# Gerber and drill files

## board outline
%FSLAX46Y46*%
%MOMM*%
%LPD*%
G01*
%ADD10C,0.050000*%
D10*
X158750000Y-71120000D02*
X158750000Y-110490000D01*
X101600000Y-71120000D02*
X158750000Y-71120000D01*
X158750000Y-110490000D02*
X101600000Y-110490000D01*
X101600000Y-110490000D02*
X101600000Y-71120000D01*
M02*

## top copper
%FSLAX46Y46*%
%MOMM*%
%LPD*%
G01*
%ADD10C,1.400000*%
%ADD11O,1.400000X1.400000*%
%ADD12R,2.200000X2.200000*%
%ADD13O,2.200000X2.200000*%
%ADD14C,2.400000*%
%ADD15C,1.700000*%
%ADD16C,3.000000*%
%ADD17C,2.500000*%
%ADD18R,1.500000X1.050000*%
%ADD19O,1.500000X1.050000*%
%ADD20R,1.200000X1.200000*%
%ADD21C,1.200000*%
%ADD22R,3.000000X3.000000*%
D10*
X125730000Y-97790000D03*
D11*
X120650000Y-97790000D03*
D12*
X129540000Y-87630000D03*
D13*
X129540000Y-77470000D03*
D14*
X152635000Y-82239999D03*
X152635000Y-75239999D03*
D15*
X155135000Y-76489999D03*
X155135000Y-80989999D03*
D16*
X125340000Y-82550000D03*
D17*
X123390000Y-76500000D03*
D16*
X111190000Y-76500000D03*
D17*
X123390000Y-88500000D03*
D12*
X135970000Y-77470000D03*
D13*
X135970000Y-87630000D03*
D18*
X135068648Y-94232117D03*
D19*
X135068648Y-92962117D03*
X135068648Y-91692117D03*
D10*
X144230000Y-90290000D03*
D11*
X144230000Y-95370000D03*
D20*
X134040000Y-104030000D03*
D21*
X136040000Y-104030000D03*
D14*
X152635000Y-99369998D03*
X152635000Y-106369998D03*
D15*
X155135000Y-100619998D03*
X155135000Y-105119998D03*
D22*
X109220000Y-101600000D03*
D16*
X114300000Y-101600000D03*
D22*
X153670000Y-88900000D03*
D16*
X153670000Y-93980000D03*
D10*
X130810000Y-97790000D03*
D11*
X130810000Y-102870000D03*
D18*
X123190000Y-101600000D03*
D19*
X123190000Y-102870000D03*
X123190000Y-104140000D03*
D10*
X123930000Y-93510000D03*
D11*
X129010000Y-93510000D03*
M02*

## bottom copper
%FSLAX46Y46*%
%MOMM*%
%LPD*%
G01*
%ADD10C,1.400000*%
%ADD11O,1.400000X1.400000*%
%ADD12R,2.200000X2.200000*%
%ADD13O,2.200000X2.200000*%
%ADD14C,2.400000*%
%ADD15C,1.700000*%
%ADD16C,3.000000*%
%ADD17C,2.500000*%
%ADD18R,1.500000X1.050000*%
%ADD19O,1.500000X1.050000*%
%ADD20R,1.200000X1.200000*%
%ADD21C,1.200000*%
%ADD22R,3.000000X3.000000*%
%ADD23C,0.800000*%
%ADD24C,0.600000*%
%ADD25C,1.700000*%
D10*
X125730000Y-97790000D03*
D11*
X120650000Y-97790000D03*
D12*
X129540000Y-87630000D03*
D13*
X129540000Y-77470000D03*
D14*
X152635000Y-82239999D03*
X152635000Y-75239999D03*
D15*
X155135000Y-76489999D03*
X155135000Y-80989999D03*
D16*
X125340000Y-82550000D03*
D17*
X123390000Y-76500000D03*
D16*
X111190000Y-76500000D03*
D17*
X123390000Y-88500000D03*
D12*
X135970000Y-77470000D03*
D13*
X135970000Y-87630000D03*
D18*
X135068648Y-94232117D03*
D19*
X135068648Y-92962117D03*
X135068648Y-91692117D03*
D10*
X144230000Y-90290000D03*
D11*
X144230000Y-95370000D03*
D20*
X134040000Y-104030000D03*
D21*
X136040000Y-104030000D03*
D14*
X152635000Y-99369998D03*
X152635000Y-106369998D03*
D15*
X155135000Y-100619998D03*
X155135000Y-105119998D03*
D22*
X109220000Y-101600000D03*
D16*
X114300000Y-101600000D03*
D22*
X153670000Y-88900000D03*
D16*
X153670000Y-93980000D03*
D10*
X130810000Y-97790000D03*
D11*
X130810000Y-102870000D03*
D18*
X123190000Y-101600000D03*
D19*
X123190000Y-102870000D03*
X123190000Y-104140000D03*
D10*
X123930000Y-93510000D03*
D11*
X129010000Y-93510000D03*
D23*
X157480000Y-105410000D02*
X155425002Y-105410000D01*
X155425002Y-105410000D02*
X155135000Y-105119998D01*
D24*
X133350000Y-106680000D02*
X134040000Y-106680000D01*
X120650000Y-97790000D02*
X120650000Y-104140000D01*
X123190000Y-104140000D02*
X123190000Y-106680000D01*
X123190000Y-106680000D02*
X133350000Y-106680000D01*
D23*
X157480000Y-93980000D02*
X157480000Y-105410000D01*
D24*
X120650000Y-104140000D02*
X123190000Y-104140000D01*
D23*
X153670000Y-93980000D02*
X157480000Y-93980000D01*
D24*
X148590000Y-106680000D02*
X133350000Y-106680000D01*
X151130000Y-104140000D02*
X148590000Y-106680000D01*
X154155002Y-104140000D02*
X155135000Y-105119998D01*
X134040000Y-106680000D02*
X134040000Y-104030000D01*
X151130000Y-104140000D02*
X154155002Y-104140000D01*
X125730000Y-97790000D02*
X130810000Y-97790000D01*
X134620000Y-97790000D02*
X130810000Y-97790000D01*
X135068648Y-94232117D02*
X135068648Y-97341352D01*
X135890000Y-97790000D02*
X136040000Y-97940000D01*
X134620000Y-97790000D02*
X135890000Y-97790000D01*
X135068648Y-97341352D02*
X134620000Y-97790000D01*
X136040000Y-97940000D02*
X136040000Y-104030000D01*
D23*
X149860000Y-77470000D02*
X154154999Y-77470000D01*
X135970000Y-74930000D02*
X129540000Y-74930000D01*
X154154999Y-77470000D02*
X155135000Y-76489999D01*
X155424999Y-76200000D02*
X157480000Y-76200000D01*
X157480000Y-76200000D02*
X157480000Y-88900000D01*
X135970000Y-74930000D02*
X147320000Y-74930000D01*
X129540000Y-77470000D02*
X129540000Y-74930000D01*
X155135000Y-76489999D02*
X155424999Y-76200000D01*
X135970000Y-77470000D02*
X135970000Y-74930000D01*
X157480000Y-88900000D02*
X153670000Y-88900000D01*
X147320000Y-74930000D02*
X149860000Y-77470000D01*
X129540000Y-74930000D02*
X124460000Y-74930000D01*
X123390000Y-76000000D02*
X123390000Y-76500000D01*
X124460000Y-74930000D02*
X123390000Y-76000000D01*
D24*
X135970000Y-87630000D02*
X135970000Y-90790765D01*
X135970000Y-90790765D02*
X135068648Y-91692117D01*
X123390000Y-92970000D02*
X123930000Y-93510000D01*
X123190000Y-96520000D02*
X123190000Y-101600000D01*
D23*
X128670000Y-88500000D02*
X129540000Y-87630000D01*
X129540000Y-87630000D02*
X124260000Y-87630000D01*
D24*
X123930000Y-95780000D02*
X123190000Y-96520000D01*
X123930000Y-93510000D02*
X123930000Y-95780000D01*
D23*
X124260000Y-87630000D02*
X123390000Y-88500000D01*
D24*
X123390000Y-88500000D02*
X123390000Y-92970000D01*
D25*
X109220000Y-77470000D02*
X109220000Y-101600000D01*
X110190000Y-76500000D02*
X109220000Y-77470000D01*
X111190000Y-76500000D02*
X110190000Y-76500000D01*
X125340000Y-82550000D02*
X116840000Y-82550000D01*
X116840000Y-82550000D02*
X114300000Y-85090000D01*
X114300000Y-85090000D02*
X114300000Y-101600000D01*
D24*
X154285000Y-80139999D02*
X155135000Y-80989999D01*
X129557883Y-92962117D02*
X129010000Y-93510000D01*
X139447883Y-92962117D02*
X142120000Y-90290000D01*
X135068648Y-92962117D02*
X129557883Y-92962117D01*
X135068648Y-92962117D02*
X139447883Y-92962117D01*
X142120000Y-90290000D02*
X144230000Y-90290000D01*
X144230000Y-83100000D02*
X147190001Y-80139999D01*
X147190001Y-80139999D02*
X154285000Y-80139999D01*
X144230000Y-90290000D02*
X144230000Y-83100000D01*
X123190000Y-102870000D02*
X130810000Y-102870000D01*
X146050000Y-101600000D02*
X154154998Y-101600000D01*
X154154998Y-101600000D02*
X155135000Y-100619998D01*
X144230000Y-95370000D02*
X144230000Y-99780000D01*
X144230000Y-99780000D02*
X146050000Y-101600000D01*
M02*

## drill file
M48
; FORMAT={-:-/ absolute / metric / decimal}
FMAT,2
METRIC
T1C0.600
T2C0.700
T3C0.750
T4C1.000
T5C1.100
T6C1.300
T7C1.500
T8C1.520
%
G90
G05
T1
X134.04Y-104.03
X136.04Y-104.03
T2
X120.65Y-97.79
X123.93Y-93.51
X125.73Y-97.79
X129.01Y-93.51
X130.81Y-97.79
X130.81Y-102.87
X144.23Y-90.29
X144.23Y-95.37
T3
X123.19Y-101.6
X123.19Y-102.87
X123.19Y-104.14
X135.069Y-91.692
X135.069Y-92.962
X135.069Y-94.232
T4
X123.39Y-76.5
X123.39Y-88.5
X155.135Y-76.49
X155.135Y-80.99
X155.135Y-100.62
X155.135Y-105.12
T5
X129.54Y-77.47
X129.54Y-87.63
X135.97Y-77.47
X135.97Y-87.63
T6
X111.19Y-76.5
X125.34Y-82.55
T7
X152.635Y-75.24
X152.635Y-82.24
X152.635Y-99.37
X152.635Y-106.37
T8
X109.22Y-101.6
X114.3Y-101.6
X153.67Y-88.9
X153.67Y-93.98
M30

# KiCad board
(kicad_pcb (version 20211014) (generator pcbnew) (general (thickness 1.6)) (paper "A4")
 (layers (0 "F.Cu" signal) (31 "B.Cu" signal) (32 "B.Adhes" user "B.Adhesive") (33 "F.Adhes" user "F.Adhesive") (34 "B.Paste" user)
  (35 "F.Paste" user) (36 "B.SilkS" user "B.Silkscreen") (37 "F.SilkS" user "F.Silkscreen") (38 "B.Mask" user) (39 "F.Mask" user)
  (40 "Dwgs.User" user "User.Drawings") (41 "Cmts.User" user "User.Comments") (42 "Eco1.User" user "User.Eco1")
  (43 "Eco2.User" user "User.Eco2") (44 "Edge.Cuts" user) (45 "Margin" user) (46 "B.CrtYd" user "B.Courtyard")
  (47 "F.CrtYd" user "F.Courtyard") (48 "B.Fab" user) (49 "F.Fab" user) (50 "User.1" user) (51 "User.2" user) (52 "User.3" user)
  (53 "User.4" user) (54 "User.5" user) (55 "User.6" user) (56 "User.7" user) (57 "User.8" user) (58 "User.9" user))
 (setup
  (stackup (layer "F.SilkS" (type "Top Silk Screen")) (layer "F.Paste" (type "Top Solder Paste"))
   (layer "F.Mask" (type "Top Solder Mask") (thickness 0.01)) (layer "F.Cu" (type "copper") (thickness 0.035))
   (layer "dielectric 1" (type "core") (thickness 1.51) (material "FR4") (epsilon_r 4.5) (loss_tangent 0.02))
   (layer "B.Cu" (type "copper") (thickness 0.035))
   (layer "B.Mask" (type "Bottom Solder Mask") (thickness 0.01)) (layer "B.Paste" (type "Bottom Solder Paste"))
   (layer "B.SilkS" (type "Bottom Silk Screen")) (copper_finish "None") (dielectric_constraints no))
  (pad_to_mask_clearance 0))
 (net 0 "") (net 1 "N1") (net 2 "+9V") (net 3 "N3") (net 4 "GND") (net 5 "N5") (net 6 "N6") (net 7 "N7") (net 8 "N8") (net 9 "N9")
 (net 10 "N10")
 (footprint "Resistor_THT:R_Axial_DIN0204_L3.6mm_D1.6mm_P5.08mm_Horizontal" (layer "F.Cu") (at 125.73 97.79 180)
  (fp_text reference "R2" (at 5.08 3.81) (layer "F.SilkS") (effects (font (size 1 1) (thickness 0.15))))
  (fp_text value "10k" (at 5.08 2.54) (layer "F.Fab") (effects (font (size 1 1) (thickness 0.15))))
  (pad "1" thru_hole circle (at 0 0 180) (size 1.4 1.4) (drill 0.7) (layers *.Cu *.Mask) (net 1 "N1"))
  (pad "2" thru_hole oval (at 5.08 0 180) (size 1.4 1.4) (drill 0.7) (layers *.Cu *.Mask) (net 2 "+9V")))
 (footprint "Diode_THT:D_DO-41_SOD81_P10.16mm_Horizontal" (layer "F.Cu") (at 129.54 87.63 90)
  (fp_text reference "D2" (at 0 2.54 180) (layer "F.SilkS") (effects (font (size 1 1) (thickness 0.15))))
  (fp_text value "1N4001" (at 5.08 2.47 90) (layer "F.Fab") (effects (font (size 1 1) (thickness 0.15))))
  (pad "1" thru_hole rect (at 0 0 90) (size 2.2 2.2) (drill 1.1) (layers *.Cu *.Mask) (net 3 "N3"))
  (pad "2" thru_hole oval (at 10.16 0 90) (size 2.2 2.2) (drill 1.1) (layers *.Cu *.Mask) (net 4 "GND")))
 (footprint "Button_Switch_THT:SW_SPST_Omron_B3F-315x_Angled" (layer "F.Cu") (at 155.135 76.489999 -90)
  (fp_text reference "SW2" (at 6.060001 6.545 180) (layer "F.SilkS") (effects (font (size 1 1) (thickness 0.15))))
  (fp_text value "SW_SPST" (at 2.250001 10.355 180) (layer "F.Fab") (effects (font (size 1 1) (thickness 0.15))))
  (pad "" thru_hole circle (at 5.75 2.5 90) (size 2.4 2.4) (drill 1.5) (layers *.Cu *.Mask))
  (pad "" thru_hole circle (at -1.25 2.5 90) (size 2.4 2.4) (drill 1.5) (layers *.Cu *.Mask))
  (pad "1" thru_hole circle (at 0 0 90) (size 1.7 1.7) (drill 1) (layers *.Cu *.Mask) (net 4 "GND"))
  (pad "2" thru_hole circle (at 4.5 0 90) (size 1.7 1.7) (drill 1) (layers *.Cu *.Mask) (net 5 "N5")))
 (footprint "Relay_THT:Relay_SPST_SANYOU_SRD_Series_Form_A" (layer "F.Cu") (at 125.34 82.55 180)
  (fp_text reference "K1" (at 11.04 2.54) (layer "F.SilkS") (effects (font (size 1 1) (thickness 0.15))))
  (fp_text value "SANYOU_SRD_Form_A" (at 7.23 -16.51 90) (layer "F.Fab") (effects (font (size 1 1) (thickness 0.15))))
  (pad "1" thru_hole circle (at 0 0 270) (size 3 3) (drill 1.3) (layers *.Cu *.Mask) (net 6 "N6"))
  (pad "2" thru_hole circle (at 1.95 6.05 270) (size 2.5 2.5) (drill 1) (layers *.Cu *.Mask) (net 4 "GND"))
  (pad "3" thru_hole circle (at 14.15 6.05 270) (size 3 3) (drill 1.3) (layers *.Cu *.Mask) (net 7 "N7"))
  (pad "5" thru_hole circle (at 1.95 -5.95 270) (size 2.5 2.5) (drill 1) (layers *.Cu *.Mask) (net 3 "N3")))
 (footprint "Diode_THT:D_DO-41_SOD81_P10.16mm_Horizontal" (layer "F.Cu") (at 135.97 77.47 -90)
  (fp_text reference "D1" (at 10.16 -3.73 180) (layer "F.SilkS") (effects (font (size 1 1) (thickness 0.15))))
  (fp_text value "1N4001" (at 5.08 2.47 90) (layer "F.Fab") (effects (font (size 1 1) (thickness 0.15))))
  (pad "1" thru_hole rect (at 0 0 270) (size 2.2 2.2) (drill 1.1) (layers *.Cu *.Mask) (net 4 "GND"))
  (pad "2" thru_hole oval (at 10.16 0 270) (size 2.2 2.2) (drill 1.1) (layers *.Cu *.Mask) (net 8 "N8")))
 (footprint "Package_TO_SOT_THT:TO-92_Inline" (layer "F.Cu") (at 135.068648 94.232117 90)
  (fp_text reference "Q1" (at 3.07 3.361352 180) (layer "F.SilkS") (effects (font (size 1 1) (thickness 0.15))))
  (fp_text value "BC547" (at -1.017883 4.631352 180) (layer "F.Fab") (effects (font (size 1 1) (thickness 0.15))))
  (pad "1" thru_hole rect (at 0 0 90) (size 1.05 1.5) (drill 0.75) (layers *.Cu *.Mask) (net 1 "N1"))
  (pad "2" thru_hole oval (at 1.27 0 90) (size 1.05 1.5) (drill 0.75) (layers *.Cu *.Mask) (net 5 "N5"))
  (pad "3" thru_hole oval (at 2.54 0 90) (size 1.05 1.5) (drill 0.75) (layers *.Cu *.Mask) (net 8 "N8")))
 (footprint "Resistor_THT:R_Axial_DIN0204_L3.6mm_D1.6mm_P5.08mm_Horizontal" (layer "F.Cu") (at 144.23 90.29 -90)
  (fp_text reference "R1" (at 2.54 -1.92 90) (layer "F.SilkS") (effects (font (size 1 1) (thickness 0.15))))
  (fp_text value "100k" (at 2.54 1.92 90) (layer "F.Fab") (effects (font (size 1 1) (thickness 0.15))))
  (pad "1" thru_hole circle (at 0 0 270) (size 1.4 1.4) (drill 0.7) (layers *.Cu *.Mask) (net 5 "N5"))
  (pad "2" thru_hole oval (at 5.08 0 270) (size 1.4 1.4) (drill 0.7) (layers *.Cu *.Mask) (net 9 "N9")))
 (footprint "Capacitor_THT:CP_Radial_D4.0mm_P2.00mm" (layer "F.Cu") (at 134.04 104.03)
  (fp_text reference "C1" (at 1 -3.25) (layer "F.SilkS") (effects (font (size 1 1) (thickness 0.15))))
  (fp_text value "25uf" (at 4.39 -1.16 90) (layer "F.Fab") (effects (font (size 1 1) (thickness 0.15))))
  (pad "1" thru_hole rect (at 0 0) (size 1.2 1.2) (drill 0.6) (layers *.Cu *.Mask) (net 2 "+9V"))
  (pad "2" thru_hole circle (at 2 0) (size 1.2 1.2) (drill 0.6) (layers *.Cu *.Mask) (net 1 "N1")))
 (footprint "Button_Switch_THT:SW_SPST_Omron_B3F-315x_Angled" (layer "F.Cu") (at 155.135 100.619998 -90)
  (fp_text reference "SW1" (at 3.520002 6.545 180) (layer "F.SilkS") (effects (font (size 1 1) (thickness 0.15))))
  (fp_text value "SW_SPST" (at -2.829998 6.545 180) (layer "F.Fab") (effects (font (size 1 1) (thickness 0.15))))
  (pad "" thru_hole circle (at -1.25 2.5 90) (size 2.4 2.4) (drill 1.5) (layers *.Cu *.Mask))
  (pad "" thru_hole circle (at 5.75 2.5 90) (size 2.4 2.4) (drill 1.5) (layers *.Cu *.Mask))
  (pad "1" thru_hole circle (at 0 0 90) (size 1.7 1.7) (drill 1) (layers *.Cu *.Mask) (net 9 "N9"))
  (pad "2" thru_hole circle (at 4.5 0 90) (size 1.7 1.7) (drill 1) (layers *.Cu *.Mask) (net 2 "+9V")))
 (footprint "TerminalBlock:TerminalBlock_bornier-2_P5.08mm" (layer "F.Cu") (at 109.22 101.6)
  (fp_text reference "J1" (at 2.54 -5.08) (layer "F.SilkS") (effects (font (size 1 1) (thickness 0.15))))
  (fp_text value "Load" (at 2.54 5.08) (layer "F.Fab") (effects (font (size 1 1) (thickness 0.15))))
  (pad "1" thru_hole rect (at 0 0) (size 3 3) (drill 1.52) (layers *.Cu *.Mask) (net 7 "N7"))
  (pad "2" thru_hole circle (at 5.08 0) (size 3 3) (drill 1.52) (layers *.Cu *.Mask) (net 6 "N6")))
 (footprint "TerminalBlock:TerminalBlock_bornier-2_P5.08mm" (layer "F.Cu") (at 153.67 88.9 -90)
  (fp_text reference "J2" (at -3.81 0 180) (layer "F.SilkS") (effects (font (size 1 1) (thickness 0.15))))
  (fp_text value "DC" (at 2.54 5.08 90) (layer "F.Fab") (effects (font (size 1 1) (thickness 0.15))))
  (pad "1" thru_hole rect (at 0 0 270) (size 3 3) (drill 1.52) (layers *.Cu *.Mask) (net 4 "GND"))
  (pad "2" thru_hole circle (at 5.08 0 270) (size 3 3) (drill 1.52) (layers *.Cu *.Mask) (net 2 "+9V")))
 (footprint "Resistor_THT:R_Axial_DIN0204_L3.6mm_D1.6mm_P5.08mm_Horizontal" (layer "F.Cu") (at 130.81 97.79 -90)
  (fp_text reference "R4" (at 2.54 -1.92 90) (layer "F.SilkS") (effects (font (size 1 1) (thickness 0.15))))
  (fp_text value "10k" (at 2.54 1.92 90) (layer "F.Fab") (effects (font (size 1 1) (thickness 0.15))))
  (pad "1" thru_hole circle (at 0 0 270) (size 1.4 1.4) (drill 0.7) (layers *.Cu *.Mask) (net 1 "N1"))
  (pad "2" thru_hole oval (at 5.08 0 270) (size 1.4 1.4) (drill 0.7) (layers *.Cu *.Mask) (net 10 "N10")))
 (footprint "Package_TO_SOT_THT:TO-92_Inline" (layer "F.Cu") (at 123.19 101.6 -90)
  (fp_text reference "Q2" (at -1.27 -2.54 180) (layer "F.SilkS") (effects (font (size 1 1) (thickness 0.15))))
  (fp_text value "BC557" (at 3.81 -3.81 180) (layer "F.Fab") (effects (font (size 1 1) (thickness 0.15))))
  (pad "1" thru_hole rect (at 0 0 270) (size 1.05 1.5) (drill 0.75) (layers *.Cu *.Mask) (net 3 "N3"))
  (pad "2" thru_hole oval (at 1.27 0 270) (size 1.05 1.5) (drill 0.75) (layers *.Cu *.Mask) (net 10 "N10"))
  (pad "3" thru_hole oval (at 2.54 0 270) (size 1.05 1.5) (drill 0.75) (layers *.Cu *.Mask) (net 2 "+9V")))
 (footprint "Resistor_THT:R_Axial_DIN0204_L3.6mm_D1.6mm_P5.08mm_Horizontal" (layer "F.Cu") (at 123.93 93.51)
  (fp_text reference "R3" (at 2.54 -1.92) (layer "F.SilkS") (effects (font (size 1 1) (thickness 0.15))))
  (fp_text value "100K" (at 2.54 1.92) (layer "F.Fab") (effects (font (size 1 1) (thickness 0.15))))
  (pad "1" thru_hole circle (at 0 0) (size 1.4 1.4) (drill 0.7) (layers *.Cu *.Mask) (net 3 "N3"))
  (pad "2" thru_hole oval (at 5.08 0) (size 1.4 1.4) (drill 0.7) (layers *.Cu *.Mask) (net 5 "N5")))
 (gr_line (start 158.75 71.12) (end 158.75 110.49) (layer "Edge.Cuts") (width 0.05))
 (gr_line (start 101.6 71.12) (end 158.75 71.12) (layer "Edge.Cuts") (width 0.05))
 (gr_line (start 158.75 110.49) (end 101.6 110.49) (layer "Edge.Cuts") (width 0.05))
 (gr_line (start 101.6 110.49) (end 101.6 71.12) (layer "Edge.Cuts") (width 0.05))
 (segment (start 157.48 105.41) (end 155.425002 105.41) (width 0.8) (layer "B.Cu") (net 2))
 (segment (start 155.425002 105.41) (end 155.135 105.119998) (width 0.8) (layer "B.Cu") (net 2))
 (segment (start 133.35 106.68) (end 134.04 106.68) (width 0.6) (layer "B.Cu") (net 2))
 (segment (start 120.65 97.79) (end 120.65 104.14) (width 0.6) (layer "B.Cu") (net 2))
 (segment (start 123.19 104.14) (end 123.19 106.68) (width 0.6) (layer "B.Cu") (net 2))
 (segment (start 123.19 106.68) (end 133.35 106.68) (width 0.6) (layer "B.Cu") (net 2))
 (segment (start 157.48 93.98) (end 157.48 105.41) (width 0.8) (layer "B.Cu") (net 2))
 (segment (start 120.65 104.14) (end 123.19 104.14) (width 0.6) (layer "B.Cu") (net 2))
 (segment (start 153.67 93.98) (end 157.48 93.98) (width 0.8) (layer "B.Cu") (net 2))
 (segment (start 148.59 106.68) (end 133.35 106.68) (width 0.6) (layer "B.Cu") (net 2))
 (segment (start 151.13 104.14) (end 148.59 106.68) (width 0.6) (layer "B.Cu") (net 2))
 (segment (start 154.155002 104.14) (end 155.135 105.119998) (width 0.6) (layer "B.Cu") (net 2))
 (segment (start 134.04 106.68) (end 134.04 104.03) (width 0.6) (layer "B.Cu") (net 2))
 (segment (start 151.13 104.14) (end 154.155002 104.14) (width 0.6) (layer "B.Cu") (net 2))
 (segment (start 125.73 97.79) (end 130.81 97.79) (width 0.6) (layer "B.Cu") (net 1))
 (segment (start 134.62 97.79) (end 130.81 97.79) (width 0.6) (layer "B.Cu") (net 1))
 (segment (start 135.068648 94.232117) (end 135.068648 97.341352) (width 0.6) (layer "B.Cu") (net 1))
 (segment (start 135.89 97.79) (end 136.04 97.94) (width 0.6) (layer "B.Cu") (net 1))
 (segment (start 134.62 97.79) (end 135.89 97.79) (width 0.6) (layer "B.Cu") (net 1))
 (segment (start 135.068648 97.341352) (end 134.62 97.79) (width 0.6) (layer "B.Cu") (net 1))
 (segment (start 136.04 97.94) (end 136.04 104.03) (width 0.6) (layer "B.Cu") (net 1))
 (segment (start 149.86 77.47) (end 154.154999 77.47) (width 0.8) (layer "B.Cu") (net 4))
 (segment (start 135.97 74.93) (end 129.54 74.93) (width 0.8) (layer "B.Cu") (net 4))
 (segment (start 154.154999 77.47) (end 155.135 76.489999) (width 0.8) (layer "B.Cu") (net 4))
 (segment (start 155.424999 76.2) (end 157.48 76.2) (width 0.8) (layer "B.Cu") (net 4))
 (segment (start 157.48 76.2) (end 157.48 88.9) (width 0.8) (layer "B.Cu") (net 4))
 (segment (start 135.97 74.93) (end 147.32 74.93) (width 0.8) (layer "B.Cu") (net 4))
 (segment (start 129.54 77.47) (end 129.54 74.93) (width 0.8) (layer "B.Cu") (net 4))
 (segment (start 155.135 76.489999) (end 155.424999 76.2) (width 0.8) (layer "B.Cu") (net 4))
 (segment (start 135.97 77.47) (end 135.97 74.93) (width 0.8) (layer "B.Cu") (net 4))
 (segment (start 157.48 88.9) (end 153.67 88.9) (width 0.8) (layer "B.Cu") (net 4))
 (segment (start 147.32 74.93) (end 149.86 77.47) (width 0.8) (layer "B.Cu") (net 4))
 (segment (start 129.54 74.93) (end 124.46 74.93) (width 0.8) (layer "B.Cu") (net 4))
 (segment (start 123.39 76) (end 123.39 76.5) (width 0.8) (layer "B.Cu") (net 4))
 (segment (start 124.46 74.93) (end 123.39 76) (width 0.8) (layer "B.Cu") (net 4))
 (segment (start 135.97 87.63) (end 135.97 90.790765) (width 0.6) (layer "B.Cu") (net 8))
 (segment (start 135.97 90.790765) (end 135.068648 91.692117) (width 0.6) (layer "B.Cu") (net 8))
 (segment (start 123.39 92.97) (end 123.93 93.51) (width 0.6) (layer "B.Cu") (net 3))
 (segment (start 123.19 96.52) (end 123.19 101.6) (width 0.6) (layer "B.Cu") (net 3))
 (segment (start 128.67 88.5) (end 129.54 87.63) (width 0.8) (layer "B.Cu") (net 3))
 (segment (start 129.54 87.63) (end 124.26 87.63) (width 0.8) (layer "B.Cu") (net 3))
 (segment (start 123.93 95.78) (end 123.19 96.52) (width 0.6) (layer "B.Cu") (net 3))
 (segment (start 123.93 93.51) (end 123.93 95.78) (width 0.6) (layer "B.Cu") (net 3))
 (segment (start 124.26 87.63) (end 123.39 88.5) (width 0.8) (layer "B.Cu") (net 3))
 (segment (start 123.39 88.5) (end 123.39 92.97) (width 0.6) (layer "B.Cu") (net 3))
 (segment (start 109.22 77.47) (end 109.22 101.6) (width 1.7) (layer "B.Cu") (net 7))
 (segment (start 110.19 76.5) (end 109.22 77.47) (width 1.7) (layer "B.Cu") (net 7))
 (segment (start 111.19 76.5) (end 110.19 76.5) (width 1.7) (layer "B.Cu") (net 7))
 (segment (start 125.34 82.55) (end 116.84 82.55) (width 1.7) (layer "B.Cu") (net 6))
 (segment (start 116.84 82.55) (end 114.3 85.09) (width 1.7) (layer "B.Cu") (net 6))
 (segment (start 114.3 85.09) (end 114.3 101.6) (width 1.7) (layer "B.Cu") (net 6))
 (segment (start 154.285 80.139999) (end 155.135 80.989999) (width 0.6) (layer "B.Cu") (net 5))
 (segment (start 129.557883 92.962117) (end 129.01 93.51) (width 0.6) (layer "B.Cu") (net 5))
 (segment (start 139.447883 92.962117) (end 142.12 90.29) (width 0.6) (layer "B.Cu") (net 5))
 (segment (start 135.068648 92.962117) (end 129.557883 92.962117) (width 0.6) (layer "B.Cu") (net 5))
 (segment (start 135.068648 92.962117) (end 139.447883 92.962117) (width 0.6) (layer "B.Cu") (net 5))
 (segment (start 142.12 90.29) (end 144.23 90.29) (width 0.6) (layer "B.Cu") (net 5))
 (segment (start 144.23 83.1) (end 147.190001 80.139999) (width 0.6) (layer "B.Cu") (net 5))
 (segment (start 147.190001 80.139999) (end 154.285 80.139999) (width 0.6) (layer "B.Cu") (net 5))
 (segment (start 144.23 90.29) (end 144.23 83.1) (width 0.6) (layer "B.Cu") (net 5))
 (segment (start 123.19 102.87) (end 130.81 102.87) (width 0.6) (layer "B.Cu") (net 10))
 (segment (start 146.05 101.6) (end 154.154998 101.6) (width 0.6) (layer "B.Cu") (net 9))
 (segment (start 154.154998 101.6) (end 155.135 100.619998) (width 0.6) (layer "B.Cu") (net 9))
 (segment (start 144.23 95.37) (end 144.23 99.78) (width 0.6) (layer "B.Cu") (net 9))
 (segment (start 144.23 99.78) (end 146.05 101.6) (width 0.6) (layer "B.Cu") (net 9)))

